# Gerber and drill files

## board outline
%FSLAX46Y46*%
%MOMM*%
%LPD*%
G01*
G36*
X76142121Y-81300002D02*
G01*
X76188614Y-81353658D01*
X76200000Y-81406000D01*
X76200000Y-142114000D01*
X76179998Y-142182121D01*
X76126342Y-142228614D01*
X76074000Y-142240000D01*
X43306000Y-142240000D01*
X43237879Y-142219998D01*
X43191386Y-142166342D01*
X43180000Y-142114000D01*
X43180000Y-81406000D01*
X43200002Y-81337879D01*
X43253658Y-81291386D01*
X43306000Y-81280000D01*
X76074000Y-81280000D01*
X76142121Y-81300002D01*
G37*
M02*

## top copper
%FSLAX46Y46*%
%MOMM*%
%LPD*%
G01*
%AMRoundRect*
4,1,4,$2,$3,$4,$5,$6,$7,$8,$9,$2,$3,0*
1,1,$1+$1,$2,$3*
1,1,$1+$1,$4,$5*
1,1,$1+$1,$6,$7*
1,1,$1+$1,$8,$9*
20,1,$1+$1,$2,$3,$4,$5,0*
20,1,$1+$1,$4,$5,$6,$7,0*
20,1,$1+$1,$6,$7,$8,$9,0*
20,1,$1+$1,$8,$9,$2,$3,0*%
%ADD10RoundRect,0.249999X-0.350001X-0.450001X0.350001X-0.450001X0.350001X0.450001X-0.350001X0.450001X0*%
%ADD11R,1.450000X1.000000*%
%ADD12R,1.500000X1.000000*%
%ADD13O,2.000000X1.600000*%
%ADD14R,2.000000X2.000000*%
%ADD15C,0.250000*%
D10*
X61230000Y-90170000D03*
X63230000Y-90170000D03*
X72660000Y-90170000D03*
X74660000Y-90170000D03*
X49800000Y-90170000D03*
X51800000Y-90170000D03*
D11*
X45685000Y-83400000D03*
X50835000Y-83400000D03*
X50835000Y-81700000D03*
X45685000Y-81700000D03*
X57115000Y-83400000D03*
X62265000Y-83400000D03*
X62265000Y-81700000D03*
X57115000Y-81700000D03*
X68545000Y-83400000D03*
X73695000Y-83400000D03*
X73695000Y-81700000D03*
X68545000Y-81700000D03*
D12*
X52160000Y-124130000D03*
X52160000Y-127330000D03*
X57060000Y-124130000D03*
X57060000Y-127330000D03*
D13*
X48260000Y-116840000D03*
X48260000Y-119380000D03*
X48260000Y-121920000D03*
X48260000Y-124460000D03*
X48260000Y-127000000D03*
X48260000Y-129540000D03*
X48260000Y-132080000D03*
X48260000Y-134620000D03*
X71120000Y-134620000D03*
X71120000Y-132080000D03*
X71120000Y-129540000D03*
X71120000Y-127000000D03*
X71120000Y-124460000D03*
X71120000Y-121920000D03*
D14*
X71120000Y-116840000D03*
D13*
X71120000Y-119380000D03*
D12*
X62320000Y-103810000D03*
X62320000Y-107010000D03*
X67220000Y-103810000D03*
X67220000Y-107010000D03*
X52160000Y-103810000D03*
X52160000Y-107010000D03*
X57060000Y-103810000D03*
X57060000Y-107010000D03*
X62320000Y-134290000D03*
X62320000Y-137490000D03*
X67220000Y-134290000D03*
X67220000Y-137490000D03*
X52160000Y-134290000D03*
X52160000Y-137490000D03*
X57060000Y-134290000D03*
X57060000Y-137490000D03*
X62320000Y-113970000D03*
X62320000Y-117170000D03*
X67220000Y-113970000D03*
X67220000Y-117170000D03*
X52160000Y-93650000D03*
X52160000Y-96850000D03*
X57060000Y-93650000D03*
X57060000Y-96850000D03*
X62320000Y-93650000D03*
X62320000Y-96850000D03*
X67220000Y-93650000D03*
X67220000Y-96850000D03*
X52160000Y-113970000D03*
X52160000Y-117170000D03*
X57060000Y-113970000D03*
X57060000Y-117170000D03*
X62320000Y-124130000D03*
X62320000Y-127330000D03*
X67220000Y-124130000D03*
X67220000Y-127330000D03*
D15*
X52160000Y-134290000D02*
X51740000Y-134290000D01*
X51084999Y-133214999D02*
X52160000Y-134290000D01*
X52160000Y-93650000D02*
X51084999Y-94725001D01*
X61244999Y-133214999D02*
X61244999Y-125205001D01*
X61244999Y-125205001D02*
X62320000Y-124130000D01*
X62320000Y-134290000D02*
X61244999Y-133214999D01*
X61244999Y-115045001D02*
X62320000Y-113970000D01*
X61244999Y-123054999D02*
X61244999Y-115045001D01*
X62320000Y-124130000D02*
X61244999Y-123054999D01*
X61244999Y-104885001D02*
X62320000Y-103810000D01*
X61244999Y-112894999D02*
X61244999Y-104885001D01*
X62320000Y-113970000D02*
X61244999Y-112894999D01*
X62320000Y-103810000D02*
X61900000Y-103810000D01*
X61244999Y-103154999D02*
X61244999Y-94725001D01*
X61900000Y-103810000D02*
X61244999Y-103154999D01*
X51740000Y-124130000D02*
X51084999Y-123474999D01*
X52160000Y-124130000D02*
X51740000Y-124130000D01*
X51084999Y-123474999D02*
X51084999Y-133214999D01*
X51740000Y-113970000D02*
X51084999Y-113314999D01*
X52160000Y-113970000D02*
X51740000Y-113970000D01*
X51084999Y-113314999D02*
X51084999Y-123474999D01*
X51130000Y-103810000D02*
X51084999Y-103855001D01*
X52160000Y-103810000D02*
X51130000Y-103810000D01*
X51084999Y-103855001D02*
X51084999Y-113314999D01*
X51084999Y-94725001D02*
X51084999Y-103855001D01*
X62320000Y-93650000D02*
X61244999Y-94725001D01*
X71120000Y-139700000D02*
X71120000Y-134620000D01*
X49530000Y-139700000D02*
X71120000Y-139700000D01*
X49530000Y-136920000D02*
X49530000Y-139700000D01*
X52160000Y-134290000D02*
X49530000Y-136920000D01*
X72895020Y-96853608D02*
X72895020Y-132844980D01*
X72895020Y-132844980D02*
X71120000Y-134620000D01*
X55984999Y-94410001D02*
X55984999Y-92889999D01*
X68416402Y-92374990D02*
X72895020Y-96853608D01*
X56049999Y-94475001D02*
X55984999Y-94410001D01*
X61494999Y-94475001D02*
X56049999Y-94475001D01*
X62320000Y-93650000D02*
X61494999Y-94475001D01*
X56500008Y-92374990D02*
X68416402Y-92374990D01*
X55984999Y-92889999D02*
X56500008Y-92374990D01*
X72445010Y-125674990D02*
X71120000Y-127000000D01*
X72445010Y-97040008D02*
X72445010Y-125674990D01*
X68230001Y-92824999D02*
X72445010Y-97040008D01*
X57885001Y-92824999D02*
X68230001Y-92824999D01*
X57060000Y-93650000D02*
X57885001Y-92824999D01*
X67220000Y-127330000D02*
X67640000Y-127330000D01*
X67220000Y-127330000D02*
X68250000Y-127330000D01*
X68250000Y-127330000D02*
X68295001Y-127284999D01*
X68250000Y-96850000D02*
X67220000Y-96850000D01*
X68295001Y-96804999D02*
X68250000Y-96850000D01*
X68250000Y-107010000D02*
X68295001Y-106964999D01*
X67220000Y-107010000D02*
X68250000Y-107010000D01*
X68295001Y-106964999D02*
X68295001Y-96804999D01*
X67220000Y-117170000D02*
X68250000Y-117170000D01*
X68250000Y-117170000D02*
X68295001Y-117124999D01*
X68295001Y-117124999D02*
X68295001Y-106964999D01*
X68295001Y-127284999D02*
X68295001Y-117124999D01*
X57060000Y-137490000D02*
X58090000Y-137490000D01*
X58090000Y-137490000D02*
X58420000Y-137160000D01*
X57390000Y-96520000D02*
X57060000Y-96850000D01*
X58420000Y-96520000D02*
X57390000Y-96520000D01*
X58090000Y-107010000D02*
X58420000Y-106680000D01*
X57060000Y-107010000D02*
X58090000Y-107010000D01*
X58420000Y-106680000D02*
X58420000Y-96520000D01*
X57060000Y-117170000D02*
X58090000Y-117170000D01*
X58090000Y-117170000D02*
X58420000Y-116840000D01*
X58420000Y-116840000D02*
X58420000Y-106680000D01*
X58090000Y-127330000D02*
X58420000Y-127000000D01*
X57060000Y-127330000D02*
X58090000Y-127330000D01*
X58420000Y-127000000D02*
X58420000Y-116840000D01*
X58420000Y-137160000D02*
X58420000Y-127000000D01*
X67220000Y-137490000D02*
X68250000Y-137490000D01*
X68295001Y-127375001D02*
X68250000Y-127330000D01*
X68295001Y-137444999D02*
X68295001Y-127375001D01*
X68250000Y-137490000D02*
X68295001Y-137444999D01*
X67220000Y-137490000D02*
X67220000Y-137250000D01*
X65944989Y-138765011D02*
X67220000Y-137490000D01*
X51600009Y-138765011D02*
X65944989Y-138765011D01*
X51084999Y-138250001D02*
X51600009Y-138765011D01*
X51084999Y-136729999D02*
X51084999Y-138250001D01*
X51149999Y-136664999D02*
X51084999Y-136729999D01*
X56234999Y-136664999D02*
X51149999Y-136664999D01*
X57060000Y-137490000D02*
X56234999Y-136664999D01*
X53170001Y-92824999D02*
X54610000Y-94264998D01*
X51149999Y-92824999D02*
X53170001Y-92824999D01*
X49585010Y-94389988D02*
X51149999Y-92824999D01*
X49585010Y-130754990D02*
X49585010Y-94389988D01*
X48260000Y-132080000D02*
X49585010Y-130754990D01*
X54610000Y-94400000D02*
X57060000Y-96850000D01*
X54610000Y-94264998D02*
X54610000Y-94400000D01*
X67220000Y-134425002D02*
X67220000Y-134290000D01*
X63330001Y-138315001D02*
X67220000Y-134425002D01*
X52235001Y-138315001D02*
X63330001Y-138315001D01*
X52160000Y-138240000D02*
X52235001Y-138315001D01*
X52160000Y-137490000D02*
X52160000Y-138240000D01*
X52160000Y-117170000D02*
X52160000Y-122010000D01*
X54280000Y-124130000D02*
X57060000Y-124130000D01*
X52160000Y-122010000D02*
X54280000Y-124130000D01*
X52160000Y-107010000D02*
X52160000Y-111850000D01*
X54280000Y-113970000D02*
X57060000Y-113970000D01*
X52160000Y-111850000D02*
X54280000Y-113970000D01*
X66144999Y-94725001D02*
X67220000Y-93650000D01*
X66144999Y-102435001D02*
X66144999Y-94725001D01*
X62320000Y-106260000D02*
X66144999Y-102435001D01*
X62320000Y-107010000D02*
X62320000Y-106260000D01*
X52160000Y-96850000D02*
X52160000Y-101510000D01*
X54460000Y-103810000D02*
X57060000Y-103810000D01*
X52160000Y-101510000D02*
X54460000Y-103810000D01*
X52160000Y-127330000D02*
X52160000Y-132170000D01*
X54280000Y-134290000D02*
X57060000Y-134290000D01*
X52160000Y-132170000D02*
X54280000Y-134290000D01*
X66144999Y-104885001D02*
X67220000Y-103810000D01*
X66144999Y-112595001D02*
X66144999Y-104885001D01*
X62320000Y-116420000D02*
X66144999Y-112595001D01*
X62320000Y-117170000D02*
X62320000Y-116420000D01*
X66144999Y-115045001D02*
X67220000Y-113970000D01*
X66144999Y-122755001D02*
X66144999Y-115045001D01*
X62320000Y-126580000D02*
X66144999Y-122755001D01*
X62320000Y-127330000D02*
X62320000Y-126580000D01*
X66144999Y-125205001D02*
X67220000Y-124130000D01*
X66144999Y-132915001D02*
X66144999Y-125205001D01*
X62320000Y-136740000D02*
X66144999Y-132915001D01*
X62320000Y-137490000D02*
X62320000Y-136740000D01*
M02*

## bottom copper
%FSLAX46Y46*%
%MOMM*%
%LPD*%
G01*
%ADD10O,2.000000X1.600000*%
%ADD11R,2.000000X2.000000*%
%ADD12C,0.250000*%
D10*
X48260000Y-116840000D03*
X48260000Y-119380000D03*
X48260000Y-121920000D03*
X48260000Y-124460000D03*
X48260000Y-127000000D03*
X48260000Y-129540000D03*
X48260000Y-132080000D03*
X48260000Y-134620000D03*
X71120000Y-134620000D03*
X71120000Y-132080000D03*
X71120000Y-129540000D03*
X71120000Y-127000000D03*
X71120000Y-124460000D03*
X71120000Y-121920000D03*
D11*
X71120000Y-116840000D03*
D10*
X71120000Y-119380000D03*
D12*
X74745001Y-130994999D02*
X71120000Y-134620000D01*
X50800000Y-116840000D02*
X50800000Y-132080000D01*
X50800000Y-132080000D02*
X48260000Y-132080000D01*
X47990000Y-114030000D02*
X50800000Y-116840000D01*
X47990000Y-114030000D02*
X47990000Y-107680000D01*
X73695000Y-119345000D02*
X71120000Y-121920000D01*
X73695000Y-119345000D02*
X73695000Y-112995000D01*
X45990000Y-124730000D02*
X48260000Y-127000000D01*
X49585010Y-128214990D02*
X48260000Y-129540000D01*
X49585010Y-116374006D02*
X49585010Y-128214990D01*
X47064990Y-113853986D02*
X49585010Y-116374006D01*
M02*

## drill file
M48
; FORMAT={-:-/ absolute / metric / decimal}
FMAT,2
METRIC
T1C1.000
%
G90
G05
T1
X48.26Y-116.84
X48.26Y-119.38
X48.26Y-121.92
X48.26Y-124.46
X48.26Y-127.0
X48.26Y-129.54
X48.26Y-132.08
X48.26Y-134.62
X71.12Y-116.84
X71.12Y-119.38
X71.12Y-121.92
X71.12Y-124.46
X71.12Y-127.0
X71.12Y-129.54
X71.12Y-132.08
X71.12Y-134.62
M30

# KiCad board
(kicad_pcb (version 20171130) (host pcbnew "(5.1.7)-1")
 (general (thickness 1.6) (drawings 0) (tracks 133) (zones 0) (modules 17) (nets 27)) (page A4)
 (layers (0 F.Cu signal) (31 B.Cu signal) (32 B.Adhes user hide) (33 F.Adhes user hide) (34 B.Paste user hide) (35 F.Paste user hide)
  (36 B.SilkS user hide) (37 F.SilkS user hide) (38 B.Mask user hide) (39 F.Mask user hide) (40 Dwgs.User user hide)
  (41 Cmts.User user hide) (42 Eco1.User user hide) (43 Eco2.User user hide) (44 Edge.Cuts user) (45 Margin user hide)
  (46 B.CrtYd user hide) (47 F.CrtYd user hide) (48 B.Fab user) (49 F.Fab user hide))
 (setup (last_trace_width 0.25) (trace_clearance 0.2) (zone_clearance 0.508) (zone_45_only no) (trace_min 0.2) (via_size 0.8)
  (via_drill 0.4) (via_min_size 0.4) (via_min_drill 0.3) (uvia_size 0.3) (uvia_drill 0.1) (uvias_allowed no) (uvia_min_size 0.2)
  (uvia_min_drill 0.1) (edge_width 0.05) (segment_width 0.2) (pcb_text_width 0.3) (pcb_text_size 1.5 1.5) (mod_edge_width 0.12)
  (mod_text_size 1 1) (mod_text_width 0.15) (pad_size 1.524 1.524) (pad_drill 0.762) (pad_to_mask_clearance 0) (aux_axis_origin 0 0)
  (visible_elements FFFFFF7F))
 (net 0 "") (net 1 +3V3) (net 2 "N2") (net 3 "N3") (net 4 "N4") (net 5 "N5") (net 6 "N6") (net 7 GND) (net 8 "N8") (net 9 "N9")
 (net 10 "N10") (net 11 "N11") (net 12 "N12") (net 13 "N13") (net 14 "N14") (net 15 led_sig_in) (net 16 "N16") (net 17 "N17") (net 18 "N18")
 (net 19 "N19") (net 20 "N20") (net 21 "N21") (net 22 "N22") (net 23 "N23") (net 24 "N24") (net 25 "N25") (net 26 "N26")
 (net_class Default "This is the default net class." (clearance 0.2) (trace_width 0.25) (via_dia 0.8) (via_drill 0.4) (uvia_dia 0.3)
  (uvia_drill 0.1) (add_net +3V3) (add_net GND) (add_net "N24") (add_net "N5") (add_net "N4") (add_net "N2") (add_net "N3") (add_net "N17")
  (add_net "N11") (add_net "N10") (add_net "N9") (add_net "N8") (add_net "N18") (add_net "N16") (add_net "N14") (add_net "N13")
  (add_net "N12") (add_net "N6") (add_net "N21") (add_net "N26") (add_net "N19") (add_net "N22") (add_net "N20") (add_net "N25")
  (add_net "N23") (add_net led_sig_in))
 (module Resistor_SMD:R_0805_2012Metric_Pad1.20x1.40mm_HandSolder (layer F.Cu) (at 62.23 90.17)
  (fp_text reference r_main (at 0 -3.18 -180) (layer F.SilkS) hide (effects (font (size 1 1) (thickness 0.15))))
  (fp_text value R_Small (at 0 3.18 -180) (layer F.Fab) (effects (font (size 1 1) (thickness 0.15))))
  (pad 1 smd roundrect (at -1 0) (size 1.2 1.4) (layers F.Cu F.Paste F.Mask) (roundrect_rratio 0.2083325))
  (pad 2 smd roundrect (at 1 0) (size 1.2 1.4) (layers F.Cu F.Paste F.Mask) (roundrect_rratio 0.2083325)))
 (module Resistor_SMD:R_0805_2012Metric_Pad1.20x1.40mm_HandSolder (layer F.Cu) (at 73.66 90.17)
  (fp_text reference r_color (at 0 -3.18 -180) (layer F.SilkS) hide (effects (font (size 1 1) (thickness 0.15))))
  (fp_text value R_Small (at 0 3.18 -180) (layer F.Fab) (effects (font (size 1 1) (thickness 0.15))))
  (pad 1 smd roundrect (at -1 0) (size 1.2 1.4) (layers F.Cu F.Paste F.Mask) (roundrect_rratio 0.2083325))
  (pad 2 smd roundrect (at 1 0) (size 1.2 1.4) (layers F.Cu F.Paste F.Mask) (roundrect_rratio 0.2083325)))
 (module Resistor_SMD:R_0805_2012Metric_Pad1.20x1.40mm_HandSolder (layer F.Cu) (at 50.8 90.17)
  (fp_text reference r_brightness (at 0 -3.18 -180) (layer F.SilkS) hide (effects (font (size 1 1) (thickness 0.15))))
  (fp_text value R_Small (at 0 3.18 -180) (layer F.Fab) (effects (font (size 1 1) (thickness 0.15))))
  (pad 1 smd roundrect (at -1 0) (size 1.2 1.4) (layers F.Cu F.Paste F.Mask) (roundrect_rratio 0.2083325))
  (pad 2 smd roundrect (at 1 0) (size 1.2 1.4) (layers F.Cu F.Paste F.Mask) (roundrect_rratio 0.2083325)))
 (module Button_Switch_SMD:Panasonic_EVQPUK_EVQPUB (layer F.Cu) (at 48.26 82.55 180)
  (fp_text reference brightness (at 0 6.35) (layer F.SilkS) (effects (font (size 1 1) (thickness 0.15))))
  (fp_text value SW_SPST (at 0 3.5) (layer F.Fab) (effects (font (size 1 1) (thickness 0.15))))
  (pad 1 smd rect (at 2.575 -0.85) (size 1.45 1) (layers F.Cu F.Paste F.Mask) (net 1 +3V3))
  (pad 1 smd rect (at -2.575 -0.85) (size 1.45 1) (layers F.Cu F.Paste F.Mask) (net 1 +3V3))
  (pad 2 smd rect (at -2.575 0.85) (size 1.45 1) (layers F.Cu F.Paste F.Mask) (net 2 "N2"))
  (pad 2 smd rect (at 2.575 0.85) (size 1.45 1) (layers F.Cu F.Paste F.Mask) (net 2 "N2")))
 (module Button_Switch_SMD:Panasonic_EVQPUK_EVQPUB (layer F.Cu) (at 59.69 82.55 180)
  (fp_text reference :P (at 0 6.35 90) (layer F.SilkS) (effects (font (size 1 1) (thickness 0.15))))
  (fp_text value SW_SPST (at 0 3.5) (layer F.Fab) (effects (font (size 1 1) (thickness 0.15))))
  (pad 1 smd rect (at 2.575 -0.85) (size 1.45 1) (layers F.Cu F.Paste F.Mask) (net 1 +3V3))
  (pad 1 smd rect (at -2.575 -0.85) (size 1.45 1) (layers F.Cu F.Paste F.Mask) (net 1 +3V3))
  (pad 2 smd rect (at -2.575 0.85) (size 1.45 1) (layers F.Cu F.Paste F.Mask) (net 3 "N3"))
  (pad 2 smd rect (at 2.575 0.85) (size 1.45 1) (layers F.Cu F.Paste F.Mask) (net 3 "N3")))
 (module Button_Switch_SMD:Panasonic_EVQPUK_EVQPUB (layer F.Cu) (at 71.12 82.55 180)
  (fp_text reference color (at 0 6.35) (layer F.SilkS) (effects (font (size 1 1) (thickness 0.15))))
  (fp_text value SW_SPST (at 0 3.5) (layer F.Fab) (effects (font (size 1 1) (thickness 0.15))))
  (pad 1 smd rect (at 2.575 -0.85) (size 1.45 1) (layers F.Cu F.Paste F.Mask) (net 1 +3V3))
  (pad 1 smd rect (at -2.575 -0.85) (size 1.45 1) (layers F.Cu F.Paste F.Mask) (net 1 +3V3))
  (pad 2 smd rect (at -2.575 0.85) (size 1.45 1) (layers F.Cu F.Paste F.Mask) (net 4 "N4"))
  (pad 2 smd rect (at 2.575 0.85) (size 1.45 1) (layers F.Cu F.Paste F.Mask) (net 4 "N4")))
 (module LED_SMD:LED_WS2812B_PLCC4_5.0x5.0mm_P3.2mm (layer F.Cu) (at 54.61 125.73)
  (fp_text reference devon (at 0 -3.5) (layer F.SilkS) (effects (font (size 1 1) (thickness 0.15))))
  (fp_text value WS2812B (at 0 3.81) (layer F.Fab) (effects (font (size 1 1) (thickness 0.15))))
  (pad 1 smd rect (at -2.45 -1.6) (size 1.5 1) (layers F.Cu F.Paste F.Mask) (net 1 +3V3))
  (pad 2 smd rect (at -2.45 1.6) (size 1.5 1) (layers F.Cu F.Paste F.Mask) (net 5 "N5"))
  (pad 4 smd rect (at 2.45 -1.6) (size 1.5 1) (layers F.Cu F.Paste F.Mask) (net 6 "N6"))
  (pad 3 smd rect (at 2.45 1.6) (size 1.5 1) (layers F.Cu F.Paste F.Mask) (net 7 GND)))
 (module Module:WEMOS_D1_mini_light (layer B.Cu) (at 71.12 116.84 180)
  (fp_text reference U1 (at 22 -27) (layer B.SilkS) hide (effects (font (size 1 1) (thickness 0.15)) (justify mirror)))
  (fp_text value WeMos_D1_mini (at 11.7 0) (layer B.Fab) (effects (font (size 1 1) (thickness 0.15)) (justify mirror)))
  (pad 16 thru_hole oval (at 22.86 0 180) (size 2 1.6) (drill 1) (layers *.Cu *.Mask) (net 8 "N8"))
  (pad 15 thru_hole oval (at 22.86 -2.54 180) (size 2 1.6) (drill 1) (layers *.Cu *.Mask) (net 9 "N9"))
  (pad 14 thru_hole oval (at 22.86 -5.08 180) (size 2 1.6) (drill 1) (layers *.Cu *.Mask) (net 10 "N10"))
  (pad 13 thru_hole oval (at 22.86 -7.62 180) (size 2 1.6) (drill 1) (layers *.Cu *.Mask) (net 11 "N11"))
  (pad 12 thru_hole oval (at 22.86 -10.16 180) (size 2 1.6) (drill 1) (layers *.Cu *.Mask) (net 2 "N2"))
  (pad 11 thru_hole oval (at 22.86 -12.7 180) (size 2 1.6) (drill 1) (layers *.Cu *.Mask) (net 3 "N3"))
  (pad 10 thru_hole oval (at 22.86 -15.24 180) (size 2 1.6) (drill 1) (layers *.Cu *.Mask) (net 7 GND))
  (pad 9 thru_hole oval (at 22.86 -17.78 180) (size 2 1.6) (drill 1) (layers *.Cu *.Mask) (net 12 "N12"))
  (pad 8 thru_hole oval (at 0 -17.78 180) (size 2 1.6) (drill 1) (layers *.Cu *.Mask) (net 1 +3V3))
  (pad 7 thru_hole oval (at 0 -15.24 180) (size 2 1.6) (drill 1) (layers *.Cu *.Mask) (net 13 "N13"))
  (pad 6 thru_hole oval (at 0 -12.7 180) (size 2 1.6) (drill 1) (layers *.Cu *.Mask) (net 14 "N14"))
  (pad 5 thru_hole oval (at 0 -10.16 180) (size 2 1.6) (drill 1) (layers *.Cu *.Mask) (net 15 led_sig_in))
  (pad 4 thru_hole oval (at 0 -7.62 180) (size 2 1.6) (drill 1) (layers *.Cu *.Mask) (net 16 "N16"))
  (pad 3 thru_hole oval (at 0 -5.08 180) (size 2 1.6) (drill 1) (layers *.Cu *.Mask) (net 4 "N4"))
  (pad 1 thru_hole rect (at 0 0 180) (size 2 2) (drill 1) (layers *.Cu *.Mask) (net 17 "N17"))
  (pad 2 thru_hole oval (at 0 -2.54 180) (size 2 1.6) (drill 1) (layers *.Cu *.Mask) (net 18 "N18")))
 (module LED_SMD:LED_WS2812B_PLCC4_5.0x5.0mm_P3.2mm (layer F.Cu) (at 64.77 105.41)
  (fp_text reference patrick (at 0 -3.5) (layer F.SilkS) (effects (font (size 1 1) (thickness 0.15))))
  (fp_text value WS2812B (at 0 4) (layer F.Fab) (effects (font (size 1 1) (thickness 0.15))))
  (pad 1 smd rect (at -2.45 -1.6) (size 1.5 1) (layers F.Cu F.Paste F.Mask) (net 1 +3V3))
  (pad 2 smd rect (at -2.45 1.6) (size 1.5 1) (layers F.Cu F.Paste F.Mask) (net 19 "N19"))
  (pad 4 smd rect (at 2.45 -1.6) (size 1.5 1) (layers F.Cu F.Paste F.Mask) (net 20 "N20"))
  (pad 3 smd rect (at 2.45 1.6) (size 1.5 1) (layers F.Cu F.Paste F.Mask) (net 7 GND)))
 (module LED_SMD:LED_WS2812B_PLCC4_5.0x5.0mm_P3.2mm (layer F.Cu) (at 54.61 105.41)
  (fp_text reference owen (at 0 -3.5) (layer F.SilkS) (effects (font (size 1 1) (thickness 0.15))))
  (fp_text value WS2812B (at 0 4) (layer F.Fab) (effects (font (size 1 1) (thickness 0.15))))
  (pad 1 smd rect (at -2.45 -1.6) (size 1.5 1) (layers F.Cu F.Paste F.Mask) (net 1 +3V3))
  (pad 2 smd rect (at -2.45 1.6) (size 1.5 1) (layers F.Cu F.Paste F.Mask) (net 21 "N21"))
  (pad 4 smd rect (at 2.45 -1.6) (size 1.5 1) (layers F.Cu F.Paste F.Mask) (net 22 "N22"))
  (pad 3 smd rect (at 2.45 1.6) (size 1.5 1) (layers F.Cu F.Paste F.Mask) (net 7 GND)))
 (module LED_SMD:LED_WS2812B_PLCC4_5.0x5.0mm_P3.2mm (layer F.Cu) (at 64.77 135.89)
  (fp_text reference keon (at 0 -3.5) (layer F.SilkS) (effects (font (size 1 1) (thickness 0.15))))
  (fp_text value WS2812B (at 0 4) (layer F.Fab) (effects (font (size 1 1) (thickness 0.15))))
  (pad 1 smd rect (at -2.45 -1.6) (size 1.5 1) (layers F.Cu F.Paste F.Mask) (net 1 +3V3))
  (pad 2 smd rect (at -2.45 1.6) (size 1.5 1) (layers F.Cu F.Paste F.Mask) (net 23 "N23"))
  (pad 4 smd rect (at 2.45 -1.6) (size 1.5 1) (layers F.Cu F.Paste F.Mask) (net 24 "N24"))
  (pad 3 smd rect (at 2.45 1.6) (size 1.5 1) (layers F.Cu F.Paste F.Mask) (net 7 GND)))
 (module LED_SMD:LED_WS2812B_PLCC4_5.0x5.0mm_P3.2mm (layer F.Cu) (at 54.61 135.89)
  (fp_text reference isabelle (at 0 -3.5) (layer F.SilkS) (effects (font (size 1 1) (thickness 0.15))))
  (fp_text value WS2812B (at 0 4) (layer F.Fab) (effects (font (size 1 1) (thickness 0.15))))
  (pad 1 smd rect (at -2.45 -1.6) (size 1.5 1) (layers F.Cu F.Paste F.Mask) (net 1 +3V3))
  (pad 2 smd rect (at -2.45 1.6) (size 1.5 1) (layers F.Cu F.Paste F.Mask) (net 24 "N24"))
  (pad 4 smd rect (at 2.45 -1.6) (size 1.5 1) (layers F.Cu F.Paste F.Mask) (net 5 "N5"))
  (pad 3 smd rect (at 2.45 1.6) (size 1.5 1) (layers F.Cu F.Paste F.Mask) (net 7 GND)))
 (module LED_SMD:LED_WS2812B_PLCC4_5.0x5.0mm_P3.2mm (layer F.Cu) (at 64.77 115.57)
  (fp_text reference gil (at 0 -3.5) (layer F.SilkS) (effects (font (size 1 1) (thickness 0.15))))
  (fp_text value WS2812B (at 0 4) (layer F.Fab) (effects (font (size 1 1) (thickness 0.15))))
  (pad 1 smd rect (at -2.45 -1.6) (size 1.5 1) (layers F.Cu F.Paste F.Mask) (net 1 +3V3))
  (pad 2 smd rect (at -2.45 1.6) (size 1.5 1) (layers F.Cu F.Paste F.Mask) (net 20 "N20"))
  (pad 4 smd rect (at 2.45 -1.6) (size 1.5 1) (layers F.Cu F.Paste F.Mask) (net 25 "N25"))
  (pad 3 smd rect (at 2.45 1.6) (size 1.5 1) (layers F.Cu F.Paste F.Mask) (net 7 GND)))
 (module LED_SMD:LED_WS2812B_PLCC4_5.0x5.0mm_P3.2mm (layer F.Cu) (at 54.61 95.25)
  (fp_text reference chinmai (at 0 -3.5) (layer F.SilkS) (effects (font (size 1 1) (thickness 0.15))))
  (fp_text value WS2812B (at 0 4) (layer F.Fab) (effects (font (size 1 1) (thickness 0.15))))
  (pad 1 smd rect (at -2.45 -1.6) (size 1.5 1) (layers F.Cu F.Paste F.Mask) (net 1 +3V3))
  (pad 2 smd rect (at -2.45 1.6) (size 1.5 1) (layers F.Cu F.Paste F.Mask) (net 22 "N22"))
  (pad 4 smd rect (at 2.45 -1.6) (size 1.5 1) (layers F.Cu F.Paste F.Mask) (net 15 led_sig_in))
  (pad 3 smd rect (at 2.45 1.6) (size 1.5 1) (layers F.Cu F.Paste F.Mask) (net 7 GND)))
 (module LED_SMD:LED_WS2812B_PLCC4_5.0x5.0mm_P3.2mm (layer F.Cu) (at 64.77 95.25)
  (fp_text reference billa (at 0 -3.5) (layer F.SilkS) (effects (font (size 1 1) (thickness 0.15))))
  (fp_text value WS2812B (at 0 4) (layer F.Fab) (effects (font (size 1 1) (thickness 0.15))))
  (pad 1 smd rect (at -2.45 -1.6) (size 1.5 1) (layers F.Cu F.Paste F.Mask) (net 1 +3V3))
  (pad 2 smd rect (at -2.45 1.6) (size 1.5 1) (layers F.Cu F.Paste F.Mask) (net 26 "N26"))
  (pad 4 smd rect (at 2.45 -1.6) (size 1.5 1) (layers F.Cu F.Paste F.Mask) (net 19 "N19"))
  (pad 3 smd rect (at 2.45 1.6) (size 1.5 1) (layers F.Cu F.Paste F.Mask) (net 7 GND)))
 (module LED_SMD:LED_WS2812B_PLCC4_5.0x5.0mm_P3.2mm (layer F.Cu) (at 54.61 115.57)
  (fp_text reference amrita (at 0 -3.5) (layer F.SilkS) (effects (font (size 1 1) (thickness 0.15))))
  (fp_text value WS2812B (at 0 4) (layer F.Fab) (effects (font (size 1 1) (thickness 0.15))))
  (pad 1 smd rect (at -2.45 -1.6) (size 1.5 1) (layers F.Cu F.Paste F.Mask) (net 1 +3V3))
  (pad 2 smd rect (at -2.45 1.6) (size 1.5 1) (layers F.Cu F.Paste F.Mask) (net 6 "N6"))
  (pad 4 smd rect (at 2.45 -1.6) (size 1.5 1) (layers F.Cu F.Paste F.Mask) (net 21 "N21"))
  (pad 3 smd rect (at 2.45 1.6) (size 1.5 1) (layers F.Cu F.Paste F.Mask) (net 7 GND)))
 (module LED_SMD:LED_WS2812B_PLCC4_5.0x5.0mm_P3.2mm (layer F.Cu) (at 64.77 125.73)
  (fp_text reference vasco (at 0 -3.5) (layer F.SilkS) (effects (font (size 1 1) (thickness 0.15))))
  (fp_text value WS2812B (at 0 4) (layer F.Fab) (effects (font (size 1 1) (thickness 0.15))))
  (pad 1 smd rect (at -2.45 -1.6) (size 1.5 1) (layers F.Cu F.Paste F.Mask) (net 1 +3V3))
  (pad 2 smd rect (at -2.45 1.6) (size 1.5 1) (layers F.Cu F.Paste F.Mask) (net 25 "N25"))
  (pad 4 smd rect (at 2.45 -1.6) (size 1.5 1) (layers F.Cu F.Paste F.Mask) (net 23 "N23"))
  (pad 3 smd rect (at 2.45 1.6) (size 1.5 1) (layers F.Cu F.Paste F.Mask) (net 7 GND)))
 (segment (start 52.16 134.29) (end 51.74 134.29) (width 0.25) (layer F.Cu) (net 1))
 (segment (start 51.084999 133.214999) (end 52.16 134.29) (width 0.25) (layer F.Cu) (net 1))
 (segment (start 52.16 93.65) (end 51.084999 94.725001) (width 0.25) (layer F.Cu) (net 1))
 (segment (start 61.244999 133.214999) (end 61.244999 125.205001) (width 0.25) (layer F.Cu) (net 1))
 (segment (start 61.244999 125.205001) (end 62.32 124.13) (width 0.25) (layer F.Cu) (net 1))
 (segment (start 62.32 134.29) (end 61.244999 133.214999) (width 0.25) (layer F.Cu) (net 1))
 (segment (start 61.244999 115.045001) (end 62.32 113.97) (width 0.25) (layer F.Cu) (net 1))
 (segment (start 61.244999 123.054999) (end 61.244999 115.045001) (width 0.25) (layer F.Cu) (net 1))
 (segment (start 62.32 124.13) (end 61.244999 123.054999) (width 0.25) (layer F.Cu) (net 1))
 (segment (start 61.244999 104.885001) (end 62.32 103.81) (width 0.25) (layer F.Cu) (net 1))
 (segment (start 61.244999 112.894999) (end 61.244999 104.885001) (width 0.25) (layer F.Cu) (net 1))
 (segment (start 62.32 113.97) (end 61.244999 112.894999) (width 0.25) (layer F.Cu) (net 1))
 (segment (start 62.32 103.81) (end 61.9 103.81) (width 0.25) (layer F.Cu) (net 1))
 (segment (start 61.244999 103.154999) (end 61.244999 94.725001) (width 0.25) (layer F.Cu) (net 1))
 (segment (start 61.9 103.81) (end 61.244999 103.154999) (width 0.25) (layer F.Cu) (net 1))
 (segment (start 51.74 124.13) (end 51.084999 123.474999) (width 0.25) (layer F.Cu) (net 1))
 (segment (start 52.16 124.13) (end 51.74 124.13) (width 0.25) (layer F.Cu) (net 1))
 (segment (start 51.084999 123.474999) (end 51.084999 133.214999) (width 0.25) (layer F.Cu) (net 1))
 (segment (start 51.74 113.97) (end 51.084999 113.314999) (width 0.25) (layer F.Cu) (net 1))
 (segment (start 52.16 113.97) (end 51.74 113.97) (width 0.25) (layer F.Cu) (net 1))
 (segment (start 51.084999 113.314999) (end 51.084999 123.474999) (width 0.25) (layer F.Cu) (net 1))
 (segment (start 51.13 103.81) (end 51.084999 103.855001) (width 0.25) (layer F.Cu) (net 1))
 (segment (start 52.16 103.81) (end 51.13 103.81) (width 0.25) (layer F.Cu) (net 1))
 (segment (start 51.084999 103.855001) (end 51.084999 113.314999) (width 0.25) (layer F.Cu) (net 1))
 (segment (start 51.084999 94.725001) (end 51.084999 103.855001) (width 0.25) (layer F.Cu) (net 1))
 (segment (start 62.32 93.65) (end 61.244999 94.725001) (width 0.25) (layer F.Cu) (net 1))
 (segment (start 71.12 139.7) (end 71.12 134.62) (width 0.25) (layer F.Cu) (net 1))
 (segment (start 49.53 139.7) (end 71.12 139.7) (width 0.25) (layer F.Cu) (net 1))
 (segment (start 49.53 136.92) (end 49.53 139.7) (width 0.25) (layer F.Cu) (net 1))
 (segment (start 52.16 134.29) (end 49.53 136.92) (width 0.25) (layer F.Cu) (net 1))
 (segment (start 72.89502 96.853608) (end 72.89502 132.84498) (width 0.25) (layer F.Cu) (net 1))
 (segment (start 72.89502 132.84498) (end 71.12 134.62) (width 0.25) (layer F.Cu) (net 1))
 (segment (start 55.984999 94.410001) (end 55.984999 92.889999) (width 0.25) (layer F.Cu) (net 1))
 (segment (start 68.416402 92.37499) (end 72.89502 96.853608) (width 0.25) (layer F.Cu) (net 1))
 (segment (start 56.049999 94.475001) (end 55.984999 94.410001) (width 0.25) (layer F.Cu) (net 1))
 (segment (start 61.494999 94.475001) (end 56.049999 94.475001) (width 0.25) (layer F.Cu) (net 1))
 (segment (start 62.32 93.65) (end 61.494999 94.475001) (width 0.25) (layer F.Cu) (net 1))
 (segment (start 74.745001 130.994999) (end 71.12 134.62) (width 0.25) (layer B.Cu) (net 1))
 (segment (start 56.500008 92.37499) (end 68.416402 92.37499) (width 0.25) (layer F.Cu) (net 1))
 (segment (start 55.984999 92.889999) (end 56.500008 92.37499) (width 0.25) (layer F.Cu) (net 1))
 (segment (start 72.44501 125.67499) (end 71.12 127) (width 0.25) (layer F.Cu) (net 15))
 (segment (start 72.44501 97.040008) (end 72.44501 125.67499) (width 0.25) (layer F.Cu) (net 15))
 (segment (start 68.230001 92.824999) (end 72.44501 97.040008) (width 0.25) (layer F.Cu) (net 15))
 (segment (start 57.885001 92.824999) (end 68.230001 92.824999) (width 0.25) (layer F.Cu) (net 15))
 (segment (start 57.06 93.65) (end 57.885001 92.824999) (width 0.25) (layer F.Cu) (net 15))
 (segment (start 67.22 127.33) (end 67.64 127.33) (width 0.25) (layer F.Cu) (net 7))
 (segment (start 67.22 127.33) (end 68.25 127.33) (width 0.25) (layer F.Cu) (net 7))
 (segment (start 68.25 127.33) (end 68.295001 127.284999) (width 0.25) (layer F.Cu) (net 7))
 (segment (start 68.25 96.85) (end 67.22 96.85) (width 0.25) (layer F.Cu) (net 7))
 (segment (start 68.295001 96.804999) (end 68.25 96.85) (width 0.25) (layer F.Cu) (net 7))
 (segment (start 68.25 107.01) (end 68.295001 106.964999) (width 0.25) (layer F.Cu) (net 7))
 (segment (start 67.22 107.01) (end 68.25 107.01) (width 0.25) (layer F.Cu) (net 7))
 (segment (start 68.295001 106.964999) (end 68.295001 96.804999) (width 0.25) (layer F.Cu) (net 7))
 (segment (start 67.22 117.17) (end 68.25 117.17) (width 0.25) (layer F.Cu) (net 7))
 (segment (start 68.25 117.17) (end 68.295001 117.124999) (width 0.25) (layer F.Cu) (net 7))
 (segment (start 68.295001 117.124999) (end 68.295001 106.964999) (width 0.25) (layer F.Cu) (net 7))
 (segment (start 68.295001 127.284999) (end 68.295001 117.124999) (width 0.25) (layer F.Cu) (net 7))
 (segment (start 57.06 137.49) (end 58.09 137.49) (width 0.25) (layer F.Cu) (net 7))
 (segment (start 58.09 137.49) (end 58.42 137.16) (width 0.25) (layer F.Cu) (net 7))
 (segment (start 57.39 96.52) (end 57.06 96.85) (width 0.25) (layer F.Cu) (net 7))
 (segment (start 58.42 96.52) (end 57.39 96.52) (width 0.25) (layer F.Cu) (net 7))
 (segment (start 58.09 107.01) (end 58.42 106.68) (width 0.25) (layer F.Cu) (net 7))
 (segment (start 57.06 107.01) (end 58.09 107.01) (width 0.25) (layer F.Cu) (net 7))
 (segment (start 58.42 106.68) (end 58.42 96.52) (width 0.25) (layer F.Cu) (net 7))
 (segment (start 57.06 117.17) (end 58.09 117.17) (width 0.25) (layer F.Cu) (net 7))
 (segment (start 58.09 117.17) (end 58.42 116.84) (width 0.25) (layer F.Cu) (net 7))
 (segment (start 58.42 116.84) (end 58.42 106.68) (width 0.25) (layer F.Cu) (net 7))
 (segment (start 58.09 127.33) (end 58.42 127) (width 0.25) (layer F.Cu) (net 7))
 (segment (start 57.06 127.33) (end 58.09 127.33) (width 0.25) (layer F.Cu) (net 7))
 (segment (start 58.42 127) (end 58.42 116.84) (width 0.25) (layer F.Cu) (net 7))
 (segment (start 58.42 137.16) (end 58.42 127) (width 0.25) (layer F.Cu) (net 7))
 (segment (start 67.22 137.49) (end 68.25 137.49) (width 0.25) (layer F.Cu) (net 7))
 (segment (start 68.295001 127.375001) (end 68.25 127.33) (width 0.25) (layer F.Cu) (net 7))
 (segment (start 68.295001 137.444999) (end 68.295001 127.375001) (width 0.25) (layer F.Cu) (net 7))
 (segment (start 68.25 137.49) (end 68.295001 137.444999) (width 0.25) (layer F.Cu) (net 7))
 (segment (start 67.22 137.49) (end 67.22 137.25) (width 0.25) (layer F.Cu) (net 7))
 (segment (start 65.944989 138.765011) (end 67.22 137.49) (width 0.25) (layer F.Cu) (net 7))
 (segment (start 51.600009 138.765011) (end 65.944989 138.765011) (width 0.25) (layer F.Cu) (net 7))
 (segment (start 51.084999 138.250001) (end 51.600009 138.765011) (width 0.25) (layer F.Cu) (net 7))
 (segment (start 51.084999 136.729999) (end 51.084999 138.250001) (width 0.25) (layer F.Cu) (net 7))
 (segment (start 51.149999 136.664999) (end 51.084999 136.729999) (width 0.25) (layer F.Cu) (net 7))
 (segment (start 56.234999 136.664999) (end 51.149999 136.664999) (width 0.25) (layer F.Cu) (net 7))
 (segment (start 57.06 137.49) (end 56.234999 136.664999) (width 0.25) (layer F.Cu) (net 7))
 (segment (start 53.170001 92.824999) (end 54.61 94.264998) (width 0.25) (layer F.Cu) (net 7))
 (segment (start 51.149999 92.824999) (end 53.170001 92.824999) (width 0.25) (layer F.Cu) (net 7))
 (segment (start 49.58501 94.389988) (end 51.149999 92.824999) (width 0.25) (layer F.Cu) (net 7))
 (segment (start 49.58501 130.75499) (end 49.58501 94.389988) (width 0.25) (layer F.Cu) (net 7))
 (segment (start 48.26 132.08) (end 49.58501 130.75499) (width 0.25) (layer F.Cu) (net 7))
 (segment (start 54.61 94.4) (end 57.06 96.85) (width 0.25) (layer F.Cu) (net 7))
 (segment (start 54.61 94.264998) (end 54.61 94.4) (width 0.25) (layer F.Cu) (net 7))
 (segment (start 50.8 116.84) (end 50.8 132.08) (width 0.25) (layer B.Cu) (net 7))
 (segment (start 50.8 132.08) (end 48.26 132.08) (width 0.25) (layer B.Cu) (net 7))
 (segment (start 47.99 114.03) (end 50.8 116.84) (width 0.25) (layer B.Cu) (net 7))
 (segment (start 47.99 114.03) (end 47.99 107.68) (width 0.25) (layer B.Cu) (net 7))
 (segment (start 67.22 134.425002) (end 67.22 134.29) (width 0.25) (layer F.Cu) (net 24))
 (segment (start 63.330001 138.315001) (end 67.22 134.425002) (width 0.25) (layer F.Cu) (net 24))
 (segment (start 52.235001 138.315001) (end 63.330001 138.315001) (width 0.25) (layer F.Cu) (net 24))
 (segment (start 52.16 138.24) (end 52.235001 138.315001) (width 0.25) (layer F.Cu) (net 24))
 (segment (start 52.16 137.49) (end 52.16 138.24) (width 0.25) (layer F.Cu) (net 24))
 (segment (start 73.695 119.345) (end 71.12 121.92) (width 0.25) (layer B.Cu) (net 4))
 (segment (start 73.695 119.345) (end 73.695 112.995) (width 0.25) (layer B.Cu) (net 4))
 (segment (start 45.99 124.73) (end 48.26 127) (width 0.25) (layer B.Cu) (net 2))
 (segment (start 49.58501 128.21499) (end 48.26 129.54) (width 0.25) (layer B.Cu) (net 3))
 (segment (start 49.58501 116.374006) (end 49.58501 128.21499) (width 0.25) (layer B.Cu) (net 3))
 (segment (start 47.06499 113.853986) (end 49.58501 116.374006) (width 0.25) (layer B.Cu) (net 3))
 (segment (start 52.16 117.17) (end 52.16 122.01) (width 0.25) (layer F.Cu) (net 6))
 (segment (start 54.28 124.13) (end 57.06 124.13) (width 0.25) (layer F.Cu) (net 6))
 (segment (start 52.16 122.01) (end 54.28 124.13) (width 0.25) (layer F.Cu) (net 6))
 (segment (start 52.16 107.01) (end 52.16 111.85) (width 0.25) (layer F.Cu) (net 21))
 (segment (start 54.28 113.97) (end 57.06 113.97) (width 0.25) (layer F.Cu) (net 21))
 (segment (start 52.16 111.85) (end 54.28 113.97) (width 0.25) (layer F.Cu) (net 21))
 (segment (start 66.144999 94.725001) (end 67.22 93.65) (width 0.25) (layer F.Cu) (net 19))
 (segment (start 66.144999 102.435001) (end 66.144999 94.725001) (width 0.25) (layer F.Cu) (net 19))
 (segment (start 62.32 106.26) (end 66.144999 102.435001) (width 0.25) (layer F.Cu) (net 19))
 (segment (start 62.32 107.01) (end 62.32 106.26) (width 0.25) (layer F.Cu) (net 19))
 (segment (start 52.16 96.85) (end 52.16 101.51) (width 0.25) (layer F.Cu) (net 22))
 (segment (start 54.46 103.81) (end 57.06 103.81) (width 0.25) (layer F.Cu) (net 22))
 (segment (start 52.16 101.51) (end 54.46 103.81) (width 0.25) (layer F.Cu) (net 22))
 (segment (start 52.16 127.33) (end 52.16 132.17) (width 0.25) (layer F.Cu) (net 5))
 (segment (start 54.28 134.29) (end 57.06 134.29) (width 0.25) (layer F.Cu) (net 5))
 (segment (start 52.16 132.17) (end 54.28 134.29) (width 0.25) (layer F.Cu) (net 5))
 (segment (start 66.144999 104.885001) (end 67.22 103.81) (width 0.25) (layer F.Cu) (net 20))
 (segment (start 66.144999 112.595001) (end 66.144999 104.885001) (width 0.25) (layer F.Cu) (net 20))
 (segment (start 62.32 116.42) (end 66.144999 112.595001) (width 0.25) (layer F.Cu) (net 20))
 (segment (start 62.32 117.17) (end 62.32 116.42) (width 0.25) (layer F.Cu) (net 20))
 (segment (start 66.144999 115.045001) (end 67.22 113.97) (width 0.25) (layer F.Cu) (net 25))
 (segment (start 66.144999 122.755001) (end 66.144999 115.045001) (width 0.25) (layer F.Cu) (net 25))
 (segment (start 62.32 126.58) (end 66.144999 122.755001) (width 0.25) (layer F.Cu) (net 25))
 (segment (start 62.32 127.33) (end 62.32 126.58) (width 0.25) (layer F.Cu) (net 25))
 (segment (start 66.144999 125.205001) (end 67.22 124.13) (width 0.25) (layer F.Cu) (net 23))
 (segment (start 66.144999 132.915001) (end 66.144999 125.205001) (width 0.25) (layer F.Cu) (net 23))
 (segment (start 62.32 136.74) (end 66.144999 132.915001) (width 0.25) (layer F.Cu) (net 23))
 (segment (start 62.32 137.49) (end 62.32 136.74) (width 0.25) (layer F.Cu) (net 23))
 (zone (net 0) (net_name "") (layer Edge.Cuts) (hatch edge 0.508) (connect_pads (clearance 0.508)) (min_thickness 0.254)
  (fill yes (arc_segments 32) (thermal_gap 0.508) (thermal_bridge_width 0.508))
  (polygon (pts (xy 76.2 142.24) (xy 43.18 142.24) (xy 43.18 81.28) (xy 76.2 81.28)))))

